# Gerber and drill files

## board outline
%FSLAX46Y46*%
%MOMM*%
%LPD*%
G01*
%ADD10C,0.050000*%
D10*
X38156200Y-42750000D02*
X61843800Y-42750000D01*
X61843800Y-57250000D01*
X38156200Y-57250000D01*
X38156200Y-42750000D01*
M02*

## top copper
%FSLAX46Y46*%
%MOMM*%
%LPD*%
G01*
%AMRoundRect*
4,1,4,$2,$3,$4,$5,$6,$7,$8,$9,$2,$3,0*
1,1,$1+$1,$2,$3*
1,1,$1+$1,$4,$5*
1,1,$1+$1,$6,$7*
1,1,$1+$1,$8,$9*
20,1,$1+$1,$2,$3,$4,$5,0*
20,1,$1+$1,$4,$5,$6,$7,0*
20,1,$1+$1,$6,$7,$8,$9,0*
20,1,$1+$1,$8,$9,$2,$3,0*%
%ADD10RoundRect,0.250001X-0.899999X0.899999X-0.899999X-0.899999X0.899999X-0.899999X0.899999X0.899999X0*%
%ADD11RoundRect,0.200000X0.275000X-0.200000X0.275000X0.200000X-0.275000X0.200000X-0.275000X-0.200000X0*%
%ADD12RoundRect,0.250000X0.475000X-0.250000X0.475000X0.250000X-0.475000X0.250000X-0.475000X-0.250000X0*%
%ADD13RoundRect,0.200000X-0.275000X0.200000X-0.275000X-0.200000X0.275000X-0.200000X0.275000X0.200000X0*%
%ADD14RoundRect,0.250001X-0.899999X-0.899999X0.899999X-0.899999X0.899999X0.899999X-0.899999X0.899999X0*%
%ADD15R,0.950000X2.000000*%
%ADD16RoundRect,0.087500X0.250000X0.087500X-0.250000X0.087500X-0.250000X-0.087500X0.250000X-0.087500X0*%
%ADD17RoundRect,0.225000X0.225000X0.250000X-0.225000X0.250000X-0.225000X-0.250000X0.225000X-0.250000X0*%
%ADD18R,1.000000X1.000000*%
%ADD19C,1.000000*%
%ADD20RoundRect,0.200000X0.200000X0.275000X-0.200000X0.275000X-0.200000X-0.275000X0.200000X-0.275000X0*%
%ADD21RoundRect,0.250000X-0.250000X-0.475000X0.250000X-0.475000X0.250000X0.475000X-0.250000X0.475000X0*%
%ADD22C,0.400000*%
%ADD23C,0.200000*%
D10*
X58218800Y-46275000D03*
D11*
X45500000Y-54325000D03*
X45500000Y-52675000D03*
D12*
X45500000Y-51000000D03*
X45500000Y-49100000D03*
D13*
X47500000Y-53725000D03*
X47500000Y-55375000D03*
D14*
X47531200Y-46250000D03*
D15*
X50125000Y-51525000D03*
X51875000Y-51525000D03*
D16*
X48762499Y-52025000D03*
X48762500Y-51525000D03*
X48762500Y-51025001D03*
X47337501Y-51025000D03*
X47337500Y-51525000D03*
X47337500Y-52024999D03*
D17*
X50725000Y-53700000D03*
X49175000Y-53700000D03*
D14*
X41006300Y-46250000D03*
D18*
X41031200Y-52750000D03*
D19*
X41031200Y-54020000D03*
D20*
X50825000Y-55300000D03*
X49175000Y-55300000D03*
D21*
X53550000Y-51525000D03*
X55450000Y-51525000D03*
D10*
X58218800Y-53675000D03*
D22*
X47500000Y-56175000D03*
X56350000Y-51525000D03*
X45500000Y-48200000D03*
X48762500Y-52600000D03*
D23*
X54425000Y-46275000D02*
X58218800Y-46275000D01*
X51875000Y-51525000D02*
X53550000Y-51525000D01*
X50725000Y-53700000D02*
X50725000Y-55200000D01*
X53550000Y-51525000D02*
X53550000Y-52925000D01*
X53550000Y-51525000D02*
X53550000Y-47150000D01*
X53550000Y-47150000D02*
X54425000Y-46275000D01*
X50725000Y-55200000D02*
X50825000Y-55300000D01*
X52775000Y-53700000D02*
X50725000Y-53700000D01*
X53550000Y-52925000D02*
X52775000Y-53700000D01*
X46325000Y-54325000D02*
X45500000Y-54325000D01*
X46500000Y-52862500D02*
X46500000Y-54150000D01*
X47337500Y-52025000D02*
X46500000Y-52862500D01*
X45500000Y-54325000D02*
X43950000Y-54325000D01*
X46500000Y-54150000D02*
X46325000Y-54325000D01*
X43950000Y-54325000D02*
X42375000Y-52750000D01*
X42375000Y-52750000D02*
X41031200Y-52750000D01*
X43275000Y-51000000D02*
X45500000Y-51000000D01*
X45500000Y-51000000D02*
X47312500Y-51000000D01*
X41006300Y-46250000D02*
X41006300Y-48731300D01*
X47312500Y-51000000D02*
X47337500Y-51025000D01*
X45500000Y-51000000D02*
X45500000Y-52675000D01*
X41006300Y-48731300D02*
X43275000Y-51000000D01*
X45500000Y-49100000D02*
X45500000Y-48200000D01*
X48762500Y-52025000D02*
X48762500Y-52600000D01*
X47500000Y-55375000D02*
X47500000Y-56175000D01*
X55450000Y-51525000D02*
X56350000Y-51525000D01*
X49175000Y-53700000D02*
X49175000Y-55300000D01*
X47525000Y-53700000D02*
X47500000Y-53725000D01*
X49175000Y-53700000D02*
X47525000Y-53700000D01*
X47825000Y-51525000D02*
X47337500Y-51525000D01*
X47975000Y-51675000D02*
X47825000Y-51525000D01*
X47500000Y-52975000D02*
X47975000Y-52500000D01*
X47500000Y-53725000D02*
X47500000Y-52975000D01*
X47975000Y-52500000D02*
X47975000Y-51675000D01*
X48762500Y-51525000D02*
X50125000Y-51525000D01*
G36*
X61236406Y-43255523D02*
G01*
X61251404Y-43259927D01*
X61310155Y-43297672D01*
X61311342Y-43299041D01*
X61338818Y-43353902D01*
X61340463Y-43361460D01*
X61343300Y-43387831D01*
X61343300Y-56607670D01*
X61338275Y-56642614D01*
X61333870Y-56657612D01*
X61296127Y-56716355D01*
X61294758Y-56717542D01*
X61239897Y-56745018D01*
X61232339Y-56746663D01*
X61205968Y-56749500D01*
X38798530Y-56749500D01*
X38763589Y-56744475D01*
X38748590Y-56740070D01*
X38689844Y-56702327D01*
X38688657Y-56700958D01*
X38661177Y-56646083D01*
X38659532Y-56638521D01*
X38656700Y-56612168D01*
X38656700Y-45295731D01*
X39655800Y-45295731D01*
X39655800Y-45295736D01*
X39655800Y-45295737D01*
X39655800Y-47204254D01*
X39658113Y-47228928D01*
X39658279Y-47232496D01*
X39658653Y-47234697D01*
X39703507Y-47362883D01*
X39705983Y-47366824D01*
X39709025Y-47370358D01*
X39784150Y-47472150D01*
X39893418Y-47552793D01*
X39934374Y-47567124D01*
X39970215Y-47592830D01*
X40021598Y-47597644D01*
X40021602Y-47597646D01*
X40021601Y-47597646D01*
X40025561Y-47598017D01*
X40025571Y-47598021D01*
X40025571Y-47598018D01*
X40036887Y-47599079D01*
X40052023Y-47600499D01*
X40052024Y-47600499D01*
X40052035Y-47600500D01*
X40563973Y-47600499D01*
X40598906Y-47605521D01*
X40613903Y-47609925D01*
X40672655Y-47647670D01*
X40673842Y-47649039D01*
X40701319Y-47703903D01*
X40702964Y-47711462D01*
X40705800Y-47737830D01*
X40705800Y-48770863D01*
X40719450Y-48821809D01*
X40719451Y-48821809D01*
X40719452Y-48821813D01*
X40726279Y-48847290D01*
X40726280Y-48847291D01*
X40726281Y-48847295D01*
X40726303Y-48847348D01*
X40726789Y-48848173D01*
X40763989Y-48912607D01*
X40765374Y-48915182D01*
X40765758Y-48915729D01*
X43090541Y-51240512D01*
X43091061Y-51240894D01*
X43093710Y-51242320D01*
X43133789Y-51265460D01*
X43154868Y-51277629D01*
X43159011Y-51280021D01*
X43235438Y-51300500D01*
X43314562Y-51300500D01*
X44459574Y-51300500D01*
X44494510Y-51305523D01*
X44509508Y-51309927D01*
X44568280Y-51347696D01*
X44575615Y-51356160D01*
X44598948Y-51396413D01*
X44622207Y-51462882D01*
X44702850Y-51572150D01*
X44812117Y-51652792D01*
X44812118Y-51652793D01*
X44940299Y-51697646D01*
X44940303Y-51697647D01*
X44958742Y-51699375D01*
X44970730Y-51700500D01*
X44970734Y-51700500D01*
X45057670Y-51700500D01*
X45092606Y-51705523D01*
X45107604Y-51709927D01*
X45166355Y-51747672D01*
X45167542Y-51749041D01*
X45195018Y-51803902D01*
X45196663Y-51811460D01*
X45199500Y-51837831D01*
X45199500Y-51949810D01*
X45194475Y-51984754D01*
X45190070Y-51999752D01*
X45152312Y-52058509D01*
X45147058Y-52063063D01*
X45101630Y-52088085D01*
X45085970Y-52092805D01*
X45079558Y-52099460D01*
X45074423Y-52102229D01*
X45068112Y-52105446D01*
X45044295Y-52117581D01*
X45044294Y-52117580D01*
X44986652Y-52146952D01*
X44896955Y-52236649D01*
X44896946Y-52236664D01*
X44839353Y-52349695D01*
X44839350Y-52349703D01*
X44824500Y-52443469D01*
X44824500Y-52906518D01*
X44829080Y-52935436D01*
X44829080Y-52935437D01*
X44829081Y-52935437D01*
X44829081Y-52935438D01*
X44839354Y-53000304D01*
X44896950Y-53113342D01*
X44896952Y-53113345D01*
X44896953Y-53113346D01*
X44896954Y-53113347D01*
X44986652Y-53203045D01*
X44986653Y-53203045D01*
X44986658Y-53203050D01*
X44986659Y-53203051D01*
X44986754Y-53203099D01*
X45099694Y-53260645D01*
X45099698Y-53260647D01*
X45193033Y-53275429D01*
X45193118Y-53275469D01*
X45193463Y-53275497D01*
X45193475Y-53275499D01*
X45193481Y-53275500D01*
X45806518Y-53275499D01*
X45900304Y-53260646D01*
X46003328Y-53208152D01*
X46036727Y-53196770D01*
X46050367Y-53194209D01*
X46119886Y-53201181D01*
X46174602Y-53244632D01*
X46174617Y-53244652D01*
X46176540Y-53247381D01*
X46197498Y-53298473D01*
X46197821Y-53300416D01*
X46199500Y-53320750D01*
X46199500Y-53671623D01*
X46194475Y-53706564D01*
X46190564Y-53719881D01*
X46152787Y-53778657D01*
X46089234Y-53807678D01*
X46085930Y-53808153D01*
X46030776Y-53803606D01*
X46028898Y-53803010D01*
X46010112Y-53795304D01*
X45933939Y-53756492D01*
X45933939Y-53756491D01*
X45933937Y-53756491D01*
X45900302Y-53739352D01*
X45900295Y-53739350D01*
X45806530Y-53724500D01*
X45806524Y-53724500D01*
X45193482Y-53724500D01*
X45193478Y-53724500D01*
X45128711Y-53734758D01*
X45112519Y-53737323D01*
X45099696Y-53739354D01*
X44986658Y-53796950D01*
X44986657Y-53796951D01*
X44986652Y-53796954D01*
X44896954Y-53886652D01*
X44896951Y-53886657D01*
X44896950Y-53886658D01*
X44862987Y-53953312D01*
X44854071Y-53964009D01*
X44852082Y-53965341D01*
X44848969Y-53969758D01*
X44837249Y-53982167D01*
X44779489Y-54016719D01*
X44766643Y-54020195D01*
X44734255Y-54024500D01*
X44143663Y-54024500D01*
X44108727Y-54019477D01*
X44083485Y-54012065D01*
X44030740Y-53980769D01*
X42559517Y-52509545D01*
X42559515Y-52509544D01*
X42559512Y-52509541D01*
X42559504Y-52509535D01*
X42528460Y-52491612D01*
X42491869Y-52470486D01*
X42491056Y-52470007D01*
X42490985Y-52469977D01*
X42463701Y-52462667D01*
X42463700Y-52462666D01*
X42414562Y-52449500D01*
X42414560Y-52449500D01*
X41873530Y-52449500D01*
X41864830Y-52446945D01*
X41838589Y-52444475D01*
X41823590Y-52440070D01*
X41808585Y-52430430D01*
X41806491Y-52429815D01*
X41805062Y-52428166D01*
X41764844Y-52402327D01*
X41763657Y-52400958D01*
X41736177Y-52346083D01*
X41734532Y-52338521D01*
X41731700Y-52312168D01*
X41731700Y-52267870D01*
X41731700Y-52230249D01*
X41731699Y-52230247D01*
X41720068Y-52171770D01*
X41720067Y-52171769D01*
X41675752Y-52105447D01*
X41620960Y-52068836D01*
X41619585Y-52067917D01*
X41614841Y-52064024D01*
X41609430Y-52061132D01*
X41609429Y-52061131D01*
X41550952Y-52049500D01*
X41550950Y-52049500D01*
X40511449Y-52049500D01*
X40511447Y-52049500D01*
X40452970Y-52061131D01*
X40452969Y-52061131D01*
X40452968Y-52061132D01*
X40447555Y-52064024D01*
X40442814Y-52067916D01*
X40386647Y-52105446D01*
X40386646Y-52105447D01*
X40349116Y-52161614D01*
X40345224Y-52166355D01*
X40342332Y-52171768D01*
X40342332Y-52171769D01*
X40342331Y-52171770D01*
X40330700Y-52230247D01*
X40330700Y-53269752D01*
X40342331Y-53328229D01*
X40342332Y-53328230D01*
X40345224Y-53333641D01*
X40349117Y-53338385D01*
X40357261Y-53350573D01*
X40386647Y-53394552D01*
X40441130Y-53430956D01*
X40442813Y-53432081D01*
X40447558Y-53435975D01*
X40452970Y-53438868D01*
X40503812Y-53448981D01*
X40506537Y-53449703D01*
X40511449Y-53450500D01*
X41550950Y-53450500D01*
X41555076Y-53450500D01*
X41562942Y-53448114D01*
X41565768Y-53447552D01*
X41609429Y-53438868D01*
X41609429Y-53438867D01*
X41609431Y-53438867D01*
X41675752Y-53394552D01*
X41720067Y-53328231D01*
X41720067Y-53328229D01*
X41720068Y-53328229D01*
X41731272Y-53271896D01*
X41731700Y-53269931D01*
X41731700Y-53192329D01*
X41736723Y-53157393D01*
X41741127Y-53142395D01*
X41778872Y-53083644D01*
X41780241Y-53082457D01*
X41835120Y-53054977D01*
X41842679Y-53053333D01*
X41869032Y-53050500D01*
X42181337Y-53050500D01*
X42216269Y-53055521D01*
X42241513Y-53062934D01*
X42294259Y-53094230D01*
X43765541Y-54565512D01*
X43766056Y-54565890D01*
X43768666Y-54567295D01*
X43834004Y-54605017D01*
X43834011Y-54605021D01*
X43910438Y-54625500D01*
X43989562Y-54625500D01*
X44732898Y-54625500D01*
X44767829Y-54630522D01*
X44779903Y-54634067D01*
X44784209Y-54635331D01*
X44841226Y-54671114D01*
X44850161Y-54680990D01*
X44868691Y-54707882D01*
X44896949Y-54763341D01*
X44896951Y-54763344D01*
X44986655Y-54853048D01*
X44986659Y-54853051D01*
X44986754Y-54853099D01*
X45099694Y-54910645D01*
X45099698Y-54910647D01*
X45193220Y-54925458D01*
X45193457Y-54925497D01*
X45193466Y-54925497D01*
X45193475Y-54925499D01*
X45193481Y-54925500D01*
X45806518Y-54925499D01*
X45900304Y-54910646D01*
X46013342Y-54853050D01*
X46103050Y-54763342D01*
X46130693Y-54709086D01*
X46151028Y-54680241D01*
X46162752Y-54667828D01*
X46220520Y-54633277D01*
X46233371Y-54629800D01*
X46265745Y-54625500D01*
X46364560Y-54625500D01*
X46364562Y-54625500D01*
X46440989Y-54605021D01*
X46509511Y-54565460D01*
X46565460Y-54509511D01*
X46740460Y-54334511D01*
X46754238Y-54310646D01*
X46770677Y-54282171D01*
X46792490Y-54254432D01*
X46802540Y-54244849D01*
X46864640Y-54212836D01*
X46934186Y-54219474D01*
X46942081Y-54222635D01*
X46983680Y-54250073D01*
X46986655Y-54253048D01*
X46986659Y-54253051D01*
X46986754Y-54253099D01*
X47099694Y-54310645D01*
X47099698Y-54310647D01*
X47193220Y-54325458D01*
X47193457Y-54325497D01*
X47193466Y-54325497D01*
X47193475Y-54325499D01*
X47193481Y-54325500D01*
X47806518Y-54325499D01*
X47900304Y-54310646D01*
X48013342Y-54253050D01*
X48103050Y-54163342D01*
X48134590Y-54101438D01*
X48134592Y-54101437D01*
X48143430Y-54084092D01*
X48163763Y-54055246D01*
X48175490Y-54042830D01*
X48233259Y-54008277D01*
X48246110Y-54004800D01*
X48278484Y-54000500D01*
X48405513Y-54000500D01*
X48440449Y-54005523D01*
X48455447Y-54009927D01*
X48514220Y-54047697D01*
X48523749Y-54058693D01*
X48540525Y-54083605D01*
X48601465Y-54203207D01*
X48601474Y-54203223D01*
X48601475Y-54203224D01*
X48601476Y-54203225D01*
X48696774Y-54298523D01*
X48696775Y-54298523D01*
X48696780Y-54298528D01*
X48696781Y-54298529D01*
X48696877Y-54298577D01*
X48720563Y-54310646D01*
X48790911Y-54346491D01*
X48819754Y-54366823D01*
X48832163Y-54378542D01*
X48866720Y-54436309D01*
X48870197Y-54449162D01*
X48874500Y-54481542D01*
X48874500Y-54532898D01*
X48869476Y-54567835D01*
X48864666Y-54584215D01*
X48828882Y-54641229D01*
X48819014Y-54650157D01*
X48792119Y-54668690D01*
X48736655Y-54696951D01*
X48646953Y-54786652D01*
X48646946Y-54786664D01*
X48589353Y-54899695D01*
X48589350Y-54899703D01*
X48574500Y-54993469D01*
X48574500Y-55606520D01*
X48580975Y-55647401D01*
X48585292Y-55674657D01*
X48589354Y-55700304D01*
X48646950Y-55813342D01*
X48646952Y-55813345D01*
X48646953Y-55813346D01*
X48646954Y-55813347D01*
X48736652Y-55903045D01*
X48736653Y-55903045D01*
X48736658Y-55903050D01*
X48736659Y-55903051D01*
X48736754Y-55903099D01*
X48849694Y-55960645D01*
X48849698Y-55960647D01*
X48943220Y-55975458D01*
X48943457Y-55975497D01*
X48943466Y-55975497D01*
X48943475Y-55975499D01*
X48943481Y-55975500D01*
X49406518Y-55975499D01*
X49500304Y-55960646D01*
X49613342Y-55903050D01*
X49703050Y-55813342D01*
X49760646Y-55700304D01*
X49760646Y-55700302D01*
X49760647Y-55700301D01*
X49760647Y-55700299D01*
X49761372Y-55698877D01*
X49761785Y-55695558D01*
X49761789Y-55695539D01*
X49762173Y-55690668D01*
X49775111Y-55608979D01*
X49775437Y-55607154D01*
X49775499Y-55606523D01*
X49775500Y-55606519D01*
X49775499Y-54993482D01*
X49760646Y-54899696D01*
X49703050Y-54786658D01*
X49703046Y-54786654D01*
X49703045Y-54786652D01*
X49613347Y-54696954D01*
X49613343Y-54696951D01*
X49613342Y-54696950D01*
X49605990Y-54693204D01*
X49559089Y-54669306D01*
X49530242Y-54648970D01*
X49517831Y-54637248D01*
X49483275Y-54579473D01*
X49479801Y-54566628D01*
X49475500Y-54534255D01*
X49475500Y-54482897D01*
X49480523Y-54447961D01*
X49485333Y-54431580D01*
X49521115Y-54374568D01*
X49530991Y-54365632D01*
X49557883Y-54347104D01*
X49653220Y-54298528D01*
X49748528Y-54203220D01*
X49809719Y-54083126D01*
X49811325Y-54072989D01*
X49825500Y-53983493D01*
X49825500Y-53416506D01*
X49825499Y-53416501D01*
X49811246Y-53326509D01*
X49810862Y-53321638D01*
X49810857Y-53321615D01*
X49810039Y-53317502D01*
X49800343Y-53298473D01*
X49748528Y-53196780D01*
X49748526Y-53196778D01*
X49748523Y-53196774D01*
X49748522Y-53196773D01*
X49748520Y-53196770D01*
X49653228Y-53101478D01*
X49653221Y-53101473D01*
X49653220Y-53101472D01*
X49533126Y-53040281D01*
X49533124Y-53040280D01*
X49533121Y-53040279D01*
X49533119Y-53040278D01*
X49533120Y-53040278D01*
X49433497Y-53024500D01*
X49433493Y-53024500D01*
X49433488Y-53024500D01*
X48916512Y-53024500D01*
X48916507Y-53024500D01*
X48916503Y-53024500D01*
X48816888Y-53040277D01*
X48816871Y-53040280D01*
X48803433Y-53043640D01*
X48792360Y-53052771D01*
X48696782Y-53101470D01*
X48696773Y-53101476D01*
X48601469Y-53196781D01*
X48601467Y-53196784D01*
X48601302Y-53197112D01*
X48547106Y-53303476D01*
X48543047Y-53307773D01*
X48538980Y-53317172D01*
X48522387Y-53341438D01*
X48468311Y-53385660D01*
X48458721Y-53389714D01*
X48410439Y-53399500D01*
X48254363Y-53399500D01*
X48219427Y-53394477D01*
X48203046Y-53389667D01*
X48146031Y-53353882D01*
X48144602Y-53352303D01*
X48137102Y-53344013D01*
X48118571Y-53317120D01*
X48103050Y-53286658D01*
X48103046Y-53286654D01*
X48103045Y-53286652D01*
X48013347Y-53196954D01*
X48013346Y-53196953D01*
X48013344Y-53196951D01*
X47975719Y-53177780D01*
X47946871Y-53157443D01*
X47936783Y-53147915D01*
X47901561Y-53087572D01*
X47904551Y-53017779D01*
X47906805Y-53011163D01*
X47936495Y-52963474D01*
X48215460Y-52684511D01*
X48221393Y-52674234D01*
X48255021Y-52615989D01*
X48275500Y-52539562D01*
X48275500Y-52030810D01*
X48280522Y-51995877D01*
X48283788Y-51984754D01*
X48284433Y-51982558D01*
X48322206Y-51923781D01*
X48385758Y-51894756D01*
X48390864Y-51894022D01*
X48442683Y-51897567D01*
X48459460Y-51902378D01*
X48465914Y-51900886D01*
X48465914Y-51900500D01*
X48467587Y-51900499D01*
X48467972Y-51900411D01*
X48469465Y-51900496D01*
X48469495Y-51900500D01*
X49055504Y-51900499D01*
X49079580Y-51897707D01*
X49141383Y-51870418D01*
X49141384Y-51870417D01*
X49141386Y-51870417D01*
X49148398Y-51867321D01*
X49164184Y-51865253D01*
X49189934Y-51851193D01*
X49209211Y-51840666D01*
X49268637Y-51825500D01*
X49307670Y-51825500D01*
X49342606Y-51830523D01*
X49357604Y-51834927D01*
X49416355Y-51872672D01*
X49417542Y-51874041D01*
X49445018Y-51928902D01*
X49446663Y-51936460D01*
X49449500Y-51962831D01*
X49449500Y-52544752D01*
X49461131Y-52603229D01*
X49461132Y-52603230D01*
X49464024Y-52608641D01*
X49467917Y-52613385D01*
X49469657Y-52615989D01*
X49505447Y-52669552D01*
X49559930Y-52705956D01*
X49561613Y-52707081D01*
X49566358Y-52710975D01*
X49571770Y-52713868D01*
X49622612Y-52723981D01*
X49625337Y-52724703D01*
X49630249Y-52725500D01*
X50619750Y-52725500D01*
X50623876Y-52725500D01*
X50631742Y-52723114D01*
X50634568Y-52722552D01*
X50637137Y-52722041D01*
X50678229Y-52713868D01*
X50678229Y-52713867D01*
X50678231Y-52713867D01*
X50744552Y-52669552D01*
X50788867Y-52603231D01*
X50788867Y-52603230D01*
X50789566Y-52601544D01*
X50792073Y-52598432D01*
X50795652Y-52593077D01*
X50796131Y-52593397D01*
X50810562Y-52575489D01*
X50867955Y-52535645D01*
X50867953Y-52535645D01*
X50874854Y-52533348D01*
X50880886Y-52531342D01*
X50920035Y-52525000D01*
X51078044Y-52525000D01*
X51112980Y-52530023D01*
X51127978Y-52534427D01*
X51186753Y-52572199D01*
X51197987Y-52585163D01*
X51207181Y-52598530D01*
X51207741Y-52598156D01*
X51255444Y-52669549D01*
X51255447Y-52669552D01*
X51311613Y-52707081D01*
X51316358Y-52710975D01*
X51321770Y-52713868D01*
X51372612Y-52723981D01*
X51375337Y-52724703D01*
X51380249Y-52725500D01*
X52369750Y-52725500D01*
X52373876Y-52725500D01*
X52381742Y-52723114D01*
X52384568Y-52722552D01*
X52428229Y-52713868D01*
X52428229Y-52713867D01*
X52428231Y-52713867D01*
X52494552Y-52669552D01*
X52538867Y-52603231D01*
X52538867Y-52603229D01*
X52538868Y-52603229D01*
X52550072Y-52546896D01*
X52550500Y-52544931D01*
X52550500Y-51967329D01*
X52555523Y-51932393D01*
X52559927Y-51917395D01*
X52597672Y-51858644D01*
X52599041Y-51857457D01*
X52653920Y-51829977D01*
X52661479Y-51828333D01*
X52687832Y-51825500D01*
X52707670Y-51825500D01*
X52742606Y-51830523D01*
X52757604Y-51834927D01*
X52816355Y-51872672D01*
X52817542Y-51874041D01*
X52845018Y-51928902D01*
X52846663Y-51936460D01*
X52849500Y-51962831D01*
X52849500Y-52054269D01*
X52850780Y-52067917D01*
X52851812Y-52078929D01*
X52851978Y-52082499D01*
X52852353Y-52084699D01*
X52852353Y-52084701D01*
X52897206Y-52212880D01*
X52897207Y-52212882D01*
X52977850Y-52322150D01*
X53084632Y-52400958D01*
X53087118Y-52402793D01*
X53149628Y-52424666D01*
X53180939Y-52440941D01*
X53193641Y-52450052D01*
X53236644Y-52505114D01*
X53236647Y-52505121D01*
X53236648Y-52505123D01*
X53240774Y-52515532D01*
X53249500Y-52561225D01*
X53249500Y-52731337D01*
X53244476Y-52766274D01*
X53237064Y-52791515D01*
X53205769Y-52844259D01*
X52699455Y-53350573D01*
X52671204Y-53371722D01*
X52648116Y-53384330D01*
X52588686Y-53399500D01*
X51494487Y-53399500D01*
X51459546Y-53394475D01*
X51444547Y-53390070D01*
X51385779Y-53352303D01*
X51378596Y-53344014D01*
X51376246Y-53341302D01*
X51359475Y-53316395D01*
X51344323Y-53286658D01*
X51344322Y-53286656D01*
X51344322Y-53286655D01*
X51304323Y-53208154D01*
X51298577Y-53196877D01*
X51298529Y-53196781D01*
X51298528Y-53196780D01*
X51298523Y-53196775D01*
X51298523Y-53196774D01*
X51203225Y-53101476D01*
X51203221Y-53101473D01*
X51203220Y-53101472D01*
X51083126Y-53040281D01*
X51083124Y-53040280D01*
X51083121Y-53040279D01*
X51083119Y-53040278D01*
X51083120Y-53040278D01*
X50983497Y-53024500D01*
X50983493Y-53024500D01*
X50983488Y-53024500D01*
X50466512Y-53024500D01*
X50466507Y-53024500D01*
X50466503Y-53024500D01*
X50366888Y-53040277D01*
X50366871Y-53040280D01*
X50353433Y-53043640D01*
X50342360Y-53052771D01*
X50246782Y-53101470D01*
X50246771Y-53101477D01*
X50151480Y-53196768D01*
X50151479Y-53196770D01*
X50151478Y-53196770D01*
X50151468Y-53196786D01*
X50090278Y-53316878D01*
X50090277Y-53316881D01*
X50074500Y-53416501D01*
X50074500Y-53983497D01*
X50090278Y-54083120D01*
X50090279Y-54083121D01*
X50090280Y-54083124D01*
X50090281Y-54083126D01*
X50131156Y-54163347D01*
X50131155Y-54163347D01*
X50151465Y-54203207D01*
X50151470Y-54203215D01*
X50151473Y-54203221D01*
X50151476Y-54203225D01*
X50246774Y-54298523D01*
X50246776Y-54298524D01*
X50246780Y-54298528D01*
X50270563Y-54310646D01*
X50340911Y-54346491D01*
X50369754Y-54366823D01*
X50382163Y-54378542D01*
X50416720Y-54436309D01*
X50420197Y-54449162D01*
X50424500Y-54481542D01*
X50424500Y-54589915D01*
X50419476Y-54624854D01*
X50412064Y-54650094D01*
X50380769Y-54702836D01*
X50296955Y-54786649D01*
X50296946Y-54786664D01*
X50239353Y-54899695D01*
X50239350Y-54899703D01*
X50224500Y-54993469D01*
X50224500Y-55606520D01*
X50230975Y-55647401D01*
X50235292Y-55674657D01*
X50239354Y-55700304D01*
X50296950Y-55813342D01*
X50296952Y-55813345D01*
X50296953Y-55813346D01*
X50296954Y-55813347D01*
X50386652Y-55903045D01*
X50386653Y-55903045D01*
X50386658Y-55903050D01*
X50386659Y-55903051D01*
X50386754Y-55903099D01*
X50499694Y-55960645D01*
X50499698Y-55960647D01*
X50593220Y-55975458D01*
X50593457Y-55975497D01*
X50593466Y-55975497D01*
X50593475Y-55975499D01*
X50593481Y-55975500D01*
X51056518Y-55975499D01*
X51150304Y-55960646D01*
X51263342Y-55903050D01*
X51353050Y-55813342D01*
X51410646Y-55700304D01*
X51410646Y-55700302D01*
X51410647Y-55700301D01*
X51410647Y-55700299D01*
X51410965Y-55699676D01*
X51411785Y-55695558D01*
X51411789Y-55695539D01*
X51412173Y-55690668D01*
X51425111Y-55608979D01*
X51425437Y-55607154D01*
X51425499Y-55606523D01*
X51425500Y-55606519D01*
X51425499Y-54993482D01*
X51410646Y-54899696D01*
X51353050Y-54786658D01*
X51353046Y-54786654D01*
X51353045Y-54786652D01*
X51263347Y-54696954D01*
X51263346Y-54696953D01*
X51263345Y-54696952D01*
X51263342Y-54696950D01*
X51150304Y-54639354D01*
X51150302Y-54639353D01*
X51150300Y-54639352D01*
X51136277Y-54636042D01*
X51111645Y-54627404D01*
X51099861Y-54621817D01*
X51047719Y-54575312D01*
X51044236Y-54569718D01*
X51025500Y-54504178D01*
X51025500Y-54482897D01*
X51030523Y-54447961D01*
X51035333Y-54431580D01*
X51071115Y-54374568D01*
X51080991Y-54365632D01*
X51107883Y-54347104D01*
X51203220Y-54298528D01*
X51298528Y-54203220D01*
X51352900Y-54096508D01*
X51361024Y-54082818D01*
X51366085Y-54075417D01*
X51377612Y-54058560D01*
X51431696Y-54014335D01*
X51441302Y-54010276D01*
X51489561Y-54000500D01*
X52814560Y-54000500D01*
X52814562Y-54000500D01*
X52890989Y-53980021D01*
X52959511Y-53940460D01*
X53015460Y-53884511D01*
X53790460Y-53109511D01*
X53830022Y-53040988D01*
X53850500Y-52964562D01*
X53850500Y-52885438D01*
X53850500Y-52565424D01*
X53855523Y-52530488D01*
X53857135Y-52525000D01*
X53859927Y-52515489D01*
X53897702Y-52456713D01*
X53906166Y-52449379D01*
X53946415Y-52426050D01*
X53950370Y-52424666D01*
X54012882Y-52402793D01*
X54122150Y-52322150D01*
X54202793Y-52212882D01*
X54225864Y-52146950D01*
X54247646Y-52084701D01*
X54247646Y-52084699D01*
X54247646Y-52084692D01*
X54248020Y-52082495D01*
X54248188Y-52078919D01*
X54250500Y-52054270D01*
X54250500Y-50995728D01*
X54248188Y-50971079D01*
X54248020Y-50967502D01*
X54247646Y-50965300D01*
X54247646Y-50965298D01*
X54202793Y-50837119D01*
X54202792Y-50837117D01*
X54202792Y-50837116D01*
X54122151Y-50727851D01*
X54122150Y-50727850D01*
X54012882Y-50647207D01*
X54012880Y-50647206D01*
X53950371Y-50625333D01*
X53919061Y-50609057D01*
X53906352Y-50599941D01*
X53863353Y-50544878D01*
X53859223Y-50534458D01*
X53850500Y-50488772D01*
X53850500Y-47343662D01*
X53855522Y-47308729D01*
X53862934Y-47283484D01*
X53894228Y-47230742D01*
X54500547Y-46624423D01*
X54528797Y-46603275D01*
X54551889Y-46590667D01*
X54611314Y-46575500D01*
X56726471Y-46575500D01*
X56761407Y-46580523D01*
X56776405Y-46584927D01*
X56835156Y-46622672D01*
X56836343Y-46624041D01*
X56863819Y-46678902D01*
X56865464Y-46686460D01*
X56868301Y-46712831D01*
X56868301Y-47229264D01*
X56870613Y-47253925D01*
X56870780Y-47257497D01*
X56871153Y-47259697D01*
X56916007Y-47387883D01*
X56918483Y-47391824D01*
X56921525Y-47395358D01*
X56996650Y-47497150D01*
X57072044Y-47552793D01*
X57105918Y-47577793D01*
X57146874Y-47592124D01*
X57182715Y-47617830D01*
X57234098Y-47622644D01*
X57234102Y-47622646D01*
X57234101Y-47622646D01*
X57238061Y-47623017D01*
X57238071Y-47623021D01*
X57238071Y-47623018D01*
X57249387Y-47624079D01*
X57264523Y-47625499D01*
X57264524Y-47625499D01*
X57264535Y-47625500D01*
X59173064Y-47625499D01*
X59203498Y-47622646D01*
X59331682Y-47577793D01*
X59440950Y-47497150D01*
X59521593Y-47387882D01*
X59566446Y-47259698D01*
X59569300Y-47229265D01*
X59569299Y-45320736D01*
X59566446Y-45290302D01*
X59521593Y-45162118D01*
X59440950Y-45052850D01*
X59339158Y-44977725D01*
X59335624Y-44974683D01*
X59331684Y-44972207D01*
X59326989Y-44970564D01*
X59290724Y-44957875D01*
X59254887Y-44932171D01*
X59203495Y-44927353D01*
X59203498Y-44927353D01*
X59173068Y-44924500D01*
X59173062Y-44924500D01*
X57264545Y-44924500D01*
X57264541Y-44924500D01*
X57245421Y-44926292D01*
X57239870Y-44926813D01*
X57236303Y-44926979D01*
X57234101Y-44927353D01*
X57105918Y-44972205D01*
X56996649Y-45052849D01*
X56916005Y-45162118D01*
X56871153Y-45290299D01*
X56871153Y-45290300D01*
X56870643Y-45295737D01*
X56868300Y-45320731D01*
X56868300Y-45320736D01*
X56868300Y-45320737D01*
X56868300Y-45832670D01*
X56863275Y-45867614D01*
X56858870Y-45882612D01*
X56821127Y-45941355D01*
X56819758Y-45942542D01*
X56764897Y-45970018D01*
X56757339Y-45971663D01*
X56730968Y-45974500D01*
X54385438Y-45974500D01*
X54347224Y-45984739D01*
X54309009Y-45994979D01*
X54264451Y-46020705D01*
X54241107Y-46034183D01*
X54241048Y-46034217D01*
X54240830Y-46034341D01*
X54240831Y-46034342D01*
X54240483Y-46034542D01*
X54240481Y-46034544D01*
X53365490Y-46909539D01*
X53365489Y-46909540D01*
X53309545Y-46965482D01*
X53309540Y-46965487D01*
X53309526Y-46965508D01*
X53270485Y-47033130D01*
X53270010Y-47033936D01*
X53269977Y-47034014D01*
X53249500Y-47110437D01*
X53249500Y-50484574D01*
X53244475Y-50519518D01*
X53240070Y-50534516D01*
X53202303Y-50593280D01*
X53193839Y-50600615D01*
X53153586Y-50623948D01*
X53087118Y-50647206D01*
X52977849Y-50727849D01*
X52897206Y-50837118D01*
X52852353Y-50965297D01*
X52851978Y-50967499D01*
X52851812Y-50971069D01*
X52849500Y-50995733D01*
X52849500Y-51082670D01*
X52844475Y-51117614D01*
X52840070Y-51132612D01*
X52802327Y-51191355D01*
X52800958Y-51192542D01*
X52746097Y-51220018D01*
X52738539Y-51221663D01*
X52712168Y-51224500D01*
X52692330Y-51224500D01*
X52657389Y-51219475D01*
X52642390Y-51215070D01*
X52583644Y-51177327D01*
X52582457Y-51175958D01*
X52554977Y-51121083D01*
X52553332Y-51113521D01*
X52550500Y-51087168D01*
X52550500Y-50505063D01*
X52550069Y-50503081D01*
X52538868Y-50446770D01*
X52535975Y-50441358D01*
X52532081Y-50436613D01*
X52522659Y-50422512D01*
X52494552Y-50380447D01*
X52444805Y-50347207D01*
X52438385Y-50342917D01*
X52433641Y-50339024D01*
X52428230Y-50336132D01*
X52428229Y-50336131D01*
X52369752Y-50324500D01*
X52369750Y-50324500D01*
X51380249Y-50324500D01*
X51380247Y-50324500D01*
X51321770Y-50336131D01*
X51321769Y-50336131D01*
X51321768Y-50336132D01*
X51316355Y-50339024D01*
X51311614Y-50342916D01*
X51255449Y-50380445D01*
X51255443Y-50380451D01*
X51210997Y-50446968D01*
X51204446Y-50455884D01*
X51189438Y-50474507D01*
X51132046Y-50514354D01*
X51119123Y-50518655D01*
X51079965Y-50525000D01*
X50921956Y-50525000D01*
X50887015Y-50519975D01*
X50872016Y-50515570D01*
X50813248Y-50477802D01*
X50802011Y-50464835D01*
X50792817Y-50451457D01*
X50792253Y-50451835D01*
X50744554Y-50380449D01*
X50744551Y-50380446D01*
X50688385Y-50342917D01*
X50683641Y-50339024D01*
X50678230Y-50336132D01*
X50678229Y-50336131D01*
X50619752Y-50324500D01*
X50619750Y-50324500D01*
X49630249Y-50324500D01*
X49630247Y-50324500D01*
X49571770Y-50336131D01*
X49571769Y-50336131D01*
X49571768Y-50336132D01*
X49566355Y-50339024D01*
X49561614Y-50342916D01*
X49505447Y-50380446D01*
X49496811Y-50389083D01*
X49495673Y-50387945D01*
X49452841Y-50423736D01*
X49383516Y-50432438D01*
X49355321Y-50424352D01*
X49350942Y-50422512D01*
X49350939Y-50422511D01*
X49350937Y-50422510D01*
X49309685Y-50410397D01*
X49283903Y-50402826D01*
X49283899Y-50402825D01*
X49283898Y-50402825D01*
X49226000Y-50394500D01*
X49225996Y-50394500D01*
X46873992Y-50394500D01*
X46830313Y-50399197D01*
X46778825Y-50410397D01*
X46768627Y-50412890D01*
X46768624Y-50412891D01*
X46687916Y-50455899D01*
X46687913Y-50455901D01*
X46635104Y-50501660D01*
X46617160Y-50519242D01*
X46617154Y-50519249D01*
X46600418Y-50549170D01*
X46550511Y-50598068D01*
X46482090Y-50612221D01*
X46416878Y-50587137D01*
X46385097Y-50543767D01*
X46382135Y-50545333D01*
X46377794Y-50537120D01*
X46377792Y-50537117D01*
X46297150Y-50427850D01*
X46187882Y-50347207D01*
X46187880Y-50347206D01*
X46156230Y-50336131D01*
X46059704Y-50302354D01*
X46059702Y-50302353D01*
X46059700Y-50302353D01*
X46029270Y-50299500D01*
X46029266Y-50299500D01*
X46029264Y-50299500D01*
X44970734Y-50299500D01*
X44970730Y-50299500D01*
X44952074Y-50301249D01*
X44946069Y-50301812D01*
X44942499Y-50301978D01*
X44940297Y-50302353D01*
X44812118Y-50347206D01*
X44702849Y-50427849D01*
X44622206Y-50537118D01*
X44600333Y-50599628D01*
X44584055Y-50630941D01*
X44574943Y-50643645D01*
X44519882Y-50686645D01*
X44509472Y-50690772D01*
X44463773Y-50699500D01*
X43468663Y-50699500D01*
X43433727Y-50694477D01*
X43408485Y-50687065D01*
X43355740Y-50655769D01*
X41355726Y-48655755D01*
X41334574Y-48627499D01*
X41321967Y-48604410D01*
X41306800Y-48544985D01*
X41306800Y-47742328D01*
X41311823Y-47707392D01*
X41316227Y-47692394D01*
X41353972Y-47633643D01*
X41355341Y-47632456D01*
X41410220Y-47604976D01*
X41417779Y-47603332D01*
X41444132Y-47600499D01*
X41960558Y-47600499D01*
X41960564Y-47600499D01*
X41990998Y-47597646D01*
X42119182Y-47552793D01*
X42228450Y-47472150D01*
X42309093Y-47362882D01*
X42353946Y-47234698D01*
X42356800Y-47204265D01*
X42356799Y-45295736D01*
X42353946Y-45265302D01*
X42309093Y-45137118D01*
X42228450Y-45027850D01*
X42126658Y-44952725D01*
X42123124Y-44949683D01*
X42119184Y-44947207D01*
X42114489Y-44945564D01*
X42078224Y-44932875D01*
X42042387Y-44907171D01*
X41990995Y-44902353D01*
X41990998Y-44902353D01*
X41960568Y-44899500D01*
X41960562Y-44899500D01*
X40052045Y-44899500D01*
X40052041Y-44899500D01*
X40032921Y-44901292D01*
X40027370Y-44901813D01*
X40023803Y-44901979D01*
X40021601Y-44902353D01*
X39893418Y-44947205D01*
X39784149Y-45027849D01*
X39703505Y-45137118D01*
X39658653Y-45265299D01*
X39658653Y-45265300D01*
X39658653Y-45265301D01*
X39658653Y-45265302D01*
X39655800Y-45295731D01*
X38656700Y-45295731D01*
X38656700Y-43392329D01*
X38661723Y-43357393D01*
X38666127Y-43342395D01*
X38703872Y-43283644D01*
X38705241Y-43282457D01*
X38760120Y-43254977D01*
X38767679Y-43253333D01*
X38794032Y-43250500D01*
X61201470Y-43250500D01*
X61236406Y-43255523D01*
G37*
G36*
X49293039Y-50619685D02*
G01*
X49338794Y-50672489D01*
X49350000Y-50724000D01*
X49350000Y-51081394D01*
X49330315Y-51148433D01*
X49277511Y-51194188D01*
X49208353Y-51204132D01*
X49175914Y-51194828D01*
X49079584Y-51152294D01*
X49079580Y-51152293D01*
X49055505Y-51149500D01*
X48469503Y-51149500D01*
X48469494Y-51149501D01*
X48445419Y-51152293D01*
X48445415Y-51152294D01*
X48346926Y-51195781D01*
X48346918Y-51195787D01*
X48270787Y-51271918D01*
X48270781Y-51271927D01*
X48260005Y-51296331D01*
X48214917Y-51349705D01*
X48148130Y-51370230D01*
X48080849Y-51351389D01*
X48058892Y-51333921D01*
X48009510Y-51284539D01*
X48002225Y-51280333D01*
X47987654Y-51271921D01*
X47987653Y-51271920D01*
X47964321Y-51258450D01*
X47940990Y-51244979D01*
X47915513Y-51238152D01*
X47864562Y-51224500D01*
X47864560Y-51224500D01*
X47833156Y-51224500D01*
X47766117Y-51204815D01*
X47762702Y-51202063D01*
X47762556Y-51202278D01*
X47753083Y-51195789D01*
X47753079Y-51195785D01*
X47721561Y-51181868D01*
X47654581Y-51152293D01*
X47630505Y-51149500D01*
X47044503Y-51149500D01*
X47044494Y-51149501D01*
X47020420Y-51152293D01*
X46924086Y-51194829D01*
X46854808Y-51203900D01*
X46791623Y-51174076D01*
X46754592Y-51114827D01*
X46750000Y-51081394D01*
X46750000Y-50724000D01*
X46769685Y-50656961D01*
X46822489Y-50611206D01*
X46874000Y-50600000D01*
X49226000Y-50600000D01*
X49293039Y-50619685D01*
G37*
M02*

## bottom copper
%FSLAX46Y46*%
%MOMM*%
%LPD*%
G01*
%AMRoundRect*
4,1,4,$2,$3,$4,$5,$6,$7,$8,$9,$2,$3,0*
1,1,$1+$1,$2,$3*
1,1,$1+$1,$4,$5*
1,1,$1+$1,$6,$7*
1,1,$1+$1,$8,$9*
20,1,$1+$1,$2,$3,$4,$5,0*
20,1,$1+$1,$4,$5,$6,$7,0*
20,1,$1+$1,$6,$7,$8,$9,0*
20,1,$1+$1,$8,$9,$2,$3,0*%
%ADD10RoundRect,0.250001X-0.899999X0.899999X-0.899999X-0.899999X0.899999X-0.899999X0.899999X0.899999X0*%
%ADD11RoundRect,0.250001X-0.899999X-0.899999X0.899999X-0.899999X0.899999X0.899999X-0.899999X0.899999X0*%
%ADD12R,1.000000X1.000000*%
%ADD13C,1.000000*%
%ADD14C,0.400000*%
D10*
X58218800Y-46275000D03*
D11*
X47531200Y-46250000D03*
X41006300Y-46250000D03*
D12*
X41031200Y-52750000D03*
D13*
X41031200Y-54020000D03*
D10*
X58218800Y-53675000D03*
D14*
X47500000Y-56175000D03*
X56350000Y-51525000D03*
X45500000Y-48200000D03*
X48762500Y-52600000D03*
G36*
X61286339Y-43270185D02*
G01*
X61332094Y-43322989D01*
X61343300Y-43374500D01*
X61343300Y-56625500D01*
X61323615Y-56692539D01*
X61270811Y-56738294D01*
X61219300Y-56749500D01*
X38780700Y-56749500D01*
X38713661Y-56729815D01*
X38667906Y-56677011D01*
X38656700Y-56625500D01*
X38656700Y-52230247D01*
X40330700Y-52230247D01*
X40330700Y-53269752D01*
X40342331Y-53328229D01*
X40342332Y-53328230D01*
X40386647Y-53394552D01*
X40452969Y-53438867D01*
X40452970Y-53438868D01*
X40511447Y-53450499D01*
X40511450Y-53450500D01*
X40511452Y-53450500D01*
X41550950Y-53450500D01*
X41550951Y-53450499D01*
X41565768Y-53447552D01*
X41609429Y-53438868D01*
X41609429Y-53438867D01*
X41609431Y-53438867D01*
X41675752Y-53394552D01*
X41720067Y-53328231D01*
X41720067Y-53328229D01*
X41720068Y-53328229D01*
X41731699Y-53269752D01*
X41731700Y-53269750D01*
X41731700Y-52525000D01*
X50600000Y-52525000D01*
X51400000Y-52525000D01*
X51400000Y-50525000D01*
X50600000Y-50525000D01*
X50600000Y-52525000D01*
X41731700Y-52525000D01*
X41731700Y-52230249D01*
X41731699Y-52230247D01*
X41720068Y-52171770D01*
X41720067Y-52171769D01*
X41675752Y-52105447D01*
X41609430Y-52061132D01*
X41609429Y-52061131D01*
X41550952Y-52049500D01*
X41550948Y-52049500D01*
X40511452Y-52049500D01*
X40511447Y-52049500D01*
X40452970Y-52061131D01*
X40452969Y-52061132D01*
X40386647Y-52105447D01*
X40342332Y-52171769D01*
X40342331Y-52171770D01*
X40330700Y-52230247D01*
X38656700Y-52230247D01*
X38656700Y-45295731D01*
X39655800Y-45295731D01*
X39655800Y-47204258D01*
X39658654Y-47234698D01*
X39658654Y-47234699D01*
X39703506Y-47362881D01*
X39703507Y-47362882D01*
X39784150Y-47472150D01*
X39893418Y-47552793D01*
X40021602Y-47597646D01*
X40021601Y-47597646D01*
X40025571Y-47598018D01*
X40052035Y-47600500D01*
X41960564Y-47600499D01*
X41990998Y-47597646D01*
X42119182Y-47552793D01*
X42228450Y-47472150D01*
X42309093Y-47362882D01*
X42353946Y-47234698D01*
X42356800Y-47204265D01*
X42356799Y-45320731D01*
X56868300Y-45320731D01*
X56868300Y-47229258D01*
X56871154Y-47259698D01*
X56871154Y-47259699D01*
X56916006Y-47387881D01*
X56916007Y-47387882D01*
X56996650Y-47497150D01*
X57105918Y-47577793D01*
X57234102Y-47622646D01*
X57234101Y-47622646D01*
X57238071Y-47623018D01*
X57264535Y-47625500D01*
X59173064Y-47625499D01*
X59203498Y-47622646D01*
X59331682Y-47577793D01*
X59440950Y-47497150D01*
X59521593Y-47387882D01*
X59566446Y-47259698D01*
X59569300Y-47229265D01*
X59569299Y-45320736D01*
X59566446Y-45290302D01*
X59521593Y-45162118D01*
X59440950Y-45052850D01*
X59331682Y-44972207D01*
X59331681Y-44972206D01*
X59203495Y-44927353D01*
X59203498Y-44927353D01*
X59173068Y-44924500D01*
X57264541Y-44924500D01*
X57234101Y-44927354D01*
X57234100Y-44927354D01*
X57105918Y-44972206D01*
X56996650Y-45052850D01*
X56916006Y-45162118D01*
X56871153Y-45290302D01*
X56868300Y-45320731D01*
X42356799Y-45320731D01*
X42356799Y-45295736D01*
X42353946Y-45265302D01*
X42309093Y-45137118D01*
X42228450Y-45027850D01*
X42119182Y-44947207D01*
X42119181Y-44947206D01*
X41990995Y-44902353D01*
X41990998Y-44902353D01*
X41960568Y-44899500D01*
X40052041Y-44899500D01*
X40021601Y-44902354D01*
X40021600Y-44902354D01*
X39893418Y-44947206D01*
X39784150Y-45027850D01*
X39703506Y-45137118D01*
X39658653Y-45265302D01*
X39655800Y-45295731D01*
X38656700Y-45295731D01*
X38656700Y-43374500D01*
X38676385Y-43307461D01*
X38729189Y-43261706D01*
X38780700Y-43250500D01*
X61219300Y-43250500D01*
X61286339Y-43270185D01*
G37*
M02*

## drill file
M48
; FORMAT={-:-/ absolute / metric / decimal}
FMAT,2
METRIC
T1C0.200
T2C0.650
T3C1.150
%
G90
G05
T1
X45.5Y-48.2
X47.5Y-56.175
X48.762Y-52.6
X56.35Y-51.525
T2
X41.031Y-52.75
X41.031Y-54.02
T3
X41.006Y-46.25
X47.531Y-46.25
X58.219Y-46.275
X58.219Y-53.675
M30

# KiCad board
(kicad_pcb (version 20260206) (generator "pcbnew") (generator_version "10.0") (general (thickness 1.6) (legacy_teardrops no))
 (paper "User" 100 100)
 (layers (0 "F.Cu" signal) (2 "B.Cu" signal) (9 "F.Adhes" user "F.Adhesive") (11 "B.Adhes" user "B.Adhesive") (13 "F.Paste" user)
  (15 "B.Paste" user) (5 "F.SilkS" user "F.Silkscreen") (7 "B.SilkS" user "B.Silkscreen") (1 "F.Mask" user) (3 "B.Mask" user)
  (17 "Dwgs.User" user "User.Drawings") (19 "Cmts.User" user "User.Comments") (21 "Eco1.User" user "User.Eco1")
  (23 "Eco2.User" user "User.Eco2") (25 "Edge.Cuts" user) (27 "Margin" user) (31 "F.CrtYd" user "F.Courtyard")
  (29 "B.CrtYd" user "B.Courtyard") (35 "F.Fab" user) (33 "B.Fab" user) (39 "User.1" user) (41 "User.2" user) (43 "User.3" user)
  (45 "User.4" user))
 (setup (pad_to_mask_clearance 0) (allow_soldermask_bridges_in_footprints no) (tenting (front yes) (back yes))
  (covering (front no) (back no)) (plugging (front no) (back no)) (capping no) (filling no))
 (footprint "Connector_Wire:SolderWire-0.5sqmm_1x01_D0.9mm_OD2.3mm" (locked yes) (layer "F.Cu") (at 58.2188 46.275 -90)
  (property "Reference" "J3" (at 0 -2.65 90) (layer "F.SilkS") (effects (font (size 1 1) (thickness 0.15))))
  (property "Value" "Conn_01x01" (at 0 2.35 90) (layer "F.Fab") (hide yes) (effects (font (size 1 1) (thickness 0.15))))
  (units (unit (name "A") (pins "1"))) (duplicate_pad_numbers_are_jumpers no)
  (pad "1" thru_hole roundrect (at 0 0 270) (size 2.3 2.3) (drill 1.15) (layers "*.Cu" "*.Mask") (remove_unused_layers no)
   (roundrect_rratio 0.108696) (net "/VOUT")))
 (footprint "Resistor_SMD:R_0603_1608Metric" (layer "F.Cu") (at 45.5 53.5 90)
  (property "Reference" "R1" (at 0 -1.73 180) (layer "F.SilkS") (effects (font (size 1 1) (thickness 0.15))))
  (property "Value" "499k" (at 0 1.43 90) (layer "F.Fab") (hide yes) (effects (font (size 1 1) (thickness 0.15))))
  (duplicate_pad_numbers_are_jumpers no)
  (pad "1" smd roundrect (at -0.825 0 90) (size 0.8 0.95) (layers "F.Cu" "F.Mask" "F.Paste") (roundrect_rratio 0.25) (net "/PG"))
  (pad "2" smd roundrect (at 0.825 0 90) (size 0.8 0.95) (layers "F.Cu" "F.Mask" "F.Paste") (roundrect_rratio 0.25) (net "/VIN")))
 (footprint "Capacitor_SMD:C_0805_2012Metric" (layer "F.Cu") (at 45.5 50.05 90)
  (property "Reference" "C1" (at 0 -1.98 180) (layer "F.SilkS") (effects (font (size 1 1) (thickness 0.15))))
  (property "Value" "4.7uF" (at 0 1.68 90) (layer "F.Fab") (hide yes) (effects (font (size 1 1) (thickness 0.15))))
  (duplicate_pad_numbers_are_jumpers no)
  (pad "1" smd roundrect (at -0.95 0 90) (size 1 1.45) (layers "F.Cu" "F.Mask" "F.Paste") (roundrect_rratio 0.25) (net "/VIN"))
  (pad "2" smd roundrect (at 0.95 0 90) (size 1 1.45) (layers "F.Cu" "F.Mask" "F.Paste") (roundrect_rratio 0.25) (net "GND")))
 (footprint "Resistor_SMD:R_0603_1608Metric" (layer "F.Cu") (at 47.5 54.55 -90)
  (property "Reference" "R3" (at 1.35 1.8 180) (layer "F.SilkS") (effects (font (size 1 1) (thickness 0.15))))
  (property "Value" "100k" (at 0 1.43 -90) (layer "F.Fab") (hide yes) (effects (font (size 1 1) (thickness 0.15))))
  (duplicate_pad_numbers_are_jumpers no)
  (pad "1" smd roundrect (at -0.825 0 -90) (size 0.8 0.95) (layers "F.Cu" "F.Mask" "F.Paste") (roundrect_rratio 0.25) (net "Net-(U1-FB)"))
  (pad "2" smd roundrect (at 0.825 0 -90) (size 0.8 0.95) (layers "F.Cu" "F.Mask" "F.Paste") (roundrect_rratio 0.25) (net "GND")))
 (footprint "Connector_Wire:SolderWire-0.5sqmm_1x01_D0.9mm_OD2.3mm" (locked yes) (layer "F.Cu") (at 47.5312 46.25)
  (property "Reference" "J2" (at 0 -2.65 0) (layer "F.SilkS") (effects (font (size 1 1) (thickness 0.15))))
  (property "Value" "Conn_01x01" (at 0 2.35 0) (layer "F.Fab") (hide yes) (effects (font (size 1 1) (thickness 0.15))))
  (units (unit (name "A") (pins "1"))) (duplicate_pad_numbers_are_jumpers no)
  (pad "1" thru_hole roundrect (at 0 0) (size 2.3 2.3) (drill 1.15) (layers "*.Cu" "*.Mask") (remove_unused_layers no)
   (roundrect_rratio 0.108696) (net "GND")))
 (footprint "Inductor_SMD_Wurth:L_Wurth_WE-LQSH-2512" (layer "F.Cu") (at 51 51.525)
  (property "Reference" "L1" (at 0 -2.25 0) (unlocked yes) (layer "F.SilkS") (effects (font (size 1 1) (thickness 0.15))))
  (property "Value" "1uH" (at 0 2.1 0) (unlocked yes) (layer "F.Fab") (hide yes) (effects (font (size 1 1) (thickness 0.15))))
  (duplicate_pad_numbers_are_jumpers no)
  (pad "1" smd rect (at -0.875 0) (size 0.95 2) (layers "F.Cu" "F.Mask" "F.Paste") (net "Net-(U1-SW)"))
  (pad "2" smd rect (at 0.875 0) (size 0.95 2) (layers "F.Cu" "F.Mask" "F.Paste") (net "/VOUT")))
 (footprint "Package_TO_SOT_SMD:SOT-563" (layer "F.Cu") (at 48.05 51.525 180)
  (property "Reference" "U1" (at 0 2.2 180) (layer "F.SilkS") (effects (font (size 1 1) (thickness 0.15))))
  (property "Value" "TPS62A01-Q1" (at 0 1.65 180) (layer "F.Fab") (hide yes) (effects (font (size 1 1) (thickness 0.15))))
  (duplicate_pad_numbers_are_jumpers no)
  (pad "1" smd roundrect (at -0.712499 -0.5 180) (size 0.675 0.35) (layers "F.Cu" "F.Mask" "F.Paste") (roundrect_rratio 0.25) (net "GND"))
  (pad "2" smd roundrect (at -0.7125 0 180) (size 0.675 0.35) (layers "F.Cu" "F.Mask" "F.Paste") (roundrect_rratio 0.25) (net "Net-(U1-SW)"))
  (pad "3" smd roundrect (at -0.7125 0.499999 180) (size 0.675 0.35) (layers "F.Cu" "F.Mask" "F.Paste") (roundrect_rratio 0.25) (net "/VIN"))
  (pad "4" smd roundrect (at 0.712499 0.5 180) (size 0.675 0.35) (layers "F.Cu" "F.Mask" "F.Paste") (roundrect_rratio 0.25) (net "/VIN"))
  (pad "5" smd roundrect (at 0.7125 0 180) (size 0.675 0.35) (layers "F.Cu" "F.Mask" "F.Paste") (roundrect_rratio 0.25) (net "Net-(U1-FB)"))
  (pad "6" smd roundrect (at 0.7125 -0.499999 180) (size 0.675 0.35) (layers "F.Cu" "F.Mask" "F.Paste") (roundrect_rratio 0.25) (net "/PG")))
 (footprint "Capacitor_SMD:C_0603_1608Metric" (layer "F.Cu") (at 49.95 53.7 180)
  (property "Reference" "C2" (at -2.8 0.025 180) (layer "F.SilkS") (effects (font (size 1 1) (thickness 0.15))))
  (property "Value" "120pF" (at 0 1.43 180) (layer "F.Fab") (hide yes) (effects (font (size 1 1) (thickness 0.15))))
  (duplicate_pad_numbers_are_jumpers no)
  (pad "1" smd roundrect (at -0.775 0 180) (size 0.9 0.95) (layers "F.Cu" "F.Mask" "F.Paste") (roundrect_rratio 0.25) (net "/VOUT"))
  (pad "2" smd roundrect (at 0.775 0 180) (size 0.9 0.95) (layers "F.Cu" "F.Mask" "F.Paste") (roundrect_rratio 0.25) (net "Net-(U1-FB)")))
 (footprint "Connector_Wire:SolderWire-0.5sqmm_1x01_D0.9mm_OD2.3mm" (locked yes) (layer "F.Cu") (at 41.0063 46.25)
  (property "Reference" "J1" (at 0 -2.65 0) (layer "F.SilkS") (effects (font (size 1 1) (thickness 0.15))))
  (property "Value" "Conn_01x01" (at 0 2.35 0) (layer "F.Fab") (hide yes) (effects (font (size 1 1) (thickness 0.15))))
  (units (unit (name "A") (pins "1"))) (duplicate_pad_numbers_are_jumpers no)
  (pad "1" thru_hole roundrect (at 0 0) (size 2.3 2.3) (drill 1.15) (layers "*.Cu" "*.Mask") (remove_unused_layers no)
   (roundrect_rratio 0.108696) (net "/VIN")))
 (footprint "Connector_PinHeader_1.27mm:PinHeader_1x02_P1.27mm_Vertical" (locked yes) (layer "F.Cu") (at 41.0312 53.385)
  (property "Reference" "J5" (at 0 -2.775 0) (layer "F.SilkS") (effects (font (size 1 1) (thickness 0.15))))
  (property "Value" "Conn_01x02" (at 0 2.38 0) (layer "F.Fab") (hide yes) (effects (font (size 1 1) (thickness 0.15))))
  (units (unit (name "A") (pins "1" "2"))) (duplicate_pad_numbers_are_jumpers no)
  (pad "1" thru_hole rect (at 0 -0.635) (size 1 1) (drill 0.65) (layers "*.Cu" "*.Mask") (remove_unused_layers no) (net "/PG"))
  (pad "2" thru_hole circle (at 0 0.635) (size 1 1) (drill 0.65) (layers "*.Cu" "*.Mask") (remove_unused_layers no) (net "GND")))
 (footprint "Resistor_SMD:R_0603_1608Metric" (layer "F.Cu") (at 50 55.3 180)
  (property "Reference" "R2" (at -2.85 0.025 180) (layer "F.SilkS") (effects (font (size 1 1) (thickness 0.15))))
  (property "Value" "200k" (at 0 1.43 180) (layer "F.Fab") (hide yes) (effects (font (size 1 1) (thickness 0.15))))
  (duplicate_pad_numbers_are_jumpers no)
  (pad "1" smd roundrect (at -0.825 0 180) (size 0.8 0.95) (layers "F.Cu" "F.Mask" "F.Paste") (roundrect_rratio 0.25) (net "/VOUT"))
  (pad "2" smd roundrect (at 0.825 0 180) (size 0.8 0.95) (layers "F.Cu" "F.Mask" "F.Paste") (roundrect_rratio 0.25) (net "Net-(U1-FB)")))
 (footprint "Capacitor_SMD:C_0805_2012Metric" (layer "F.Cu") (at 54.5 51.525)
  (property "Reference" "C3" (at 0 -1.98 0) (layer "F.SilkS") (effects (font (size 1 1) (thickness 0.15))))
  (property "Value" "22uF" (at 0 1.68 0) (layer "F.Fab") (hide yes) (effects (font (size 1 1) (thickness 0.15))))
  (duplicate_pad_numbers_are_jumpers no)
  (pad "1" smd roundrect (at -0.95 0) (size 1 1.45) (layers "F.Cu" "F.Mask" "F.Paste") (roundrect_rratio 0.25) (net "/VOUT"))
  (pad "2" smd roundrect (at 0.95 0) (size 1 1.45) (layers "F.Cu" "F.Mask" "F.Paste") (roundrect_rratio 0.25) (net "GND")))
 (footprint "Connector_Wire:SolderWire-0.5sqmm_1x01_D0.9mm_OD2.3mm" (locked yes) (layer "F.Cu") (at 58.2188 53.675 -90)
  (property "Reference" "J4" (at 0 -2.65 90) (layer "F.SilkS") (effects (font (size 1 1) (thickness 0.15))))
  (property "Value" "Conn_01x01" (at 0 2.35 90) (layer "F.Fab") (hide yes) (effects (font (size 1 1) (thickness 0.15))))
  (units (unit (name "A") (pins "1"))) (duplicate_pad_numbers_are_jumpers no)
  (pad "1" thru_hole roundrect (at 0 0 270) (size 2.3 2.3) (drill 1.15) (layers "*.Cu" "*.Mask") (remove_unused_layers no)
   (roundrect_rratio 0.108696) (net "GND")))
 (gr_rect (start 38.1562 42.75) (end 61.8438 57.25) (stroke (width 0.05) (type solid)) (fill no) (locked yes) (layer "Edge.Cuts"))
 (segment (start 54.425 46.275) (end 58.2188 46.275) (width 0.2) (layer "F.Cu") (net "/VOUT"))
 (segment (start 51.875 51.525) (end 53.55 51.525) (width 0.2) (layer "F.Cu") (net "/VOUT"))
 (segment (start 50.725 53.7) (end 50.725 55.2) (width 0.2) (layer "F.Cu") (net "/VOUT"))
 (segment (start 53.55 51.525) (end 53.55 52.925) (width 0.2) (layer "F.Cu") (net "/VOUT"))
 (segment (start 53.55 51.525) (end 53.55 47.15) (width 0.2) (layer "F.Cu") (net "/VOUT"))
 (segment (start 53.55 47.15) (end 54.425 46.275) (width 0.2) (layer "F.Cu") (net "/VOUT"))
 (segment (start 50.725 55.2) (end 50.825 55.3) (width 0.2) (layer "F.Cu") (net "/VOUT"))
 (segment (start 52.775 53.7) (end 50.725 53.7) (width 0.2) (layer "F.Cu") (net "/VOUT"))
 (segment (start 53.55 52.925) (end 52.775 53.7) (width 0.2) (layer "F.Cu") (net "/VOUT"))
 (segment (start 46.325 54.325) (end 45.5 54.325) (width 0.2) (layer "F.Cu") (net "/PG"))
 (segment (start 46.5 52.8625) (end 46.5 54.15) (width 0.2) (layer "F.Cu") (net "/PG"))
 (segment (start 47.3375 52.025) (end 46.5 52.8625) (width 0.2) (layer "F.Cu") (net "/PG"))
 (segment (start 45.5 54.325) (end 43.95 54.325) (width 0.2) (layer "F.Cu") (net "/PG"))
 (segment (start 46.5 54.15) (end 46.325 54.325) (width 0.2) (layer "F.Cu") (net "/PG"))
 (segment (start 43.95 54.325) (end 42.375 52.75) (width 0.2) (layer "F.Cu") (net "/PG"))
 (segment (start 42.375 52.75) (end 41.0312 52.75) (width 0.2) (layer "F.Cu") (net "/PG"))
 (segment (start 43.275 51) (end 45.5 51) (width 0.2) (layer "F.Cu") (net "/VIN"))
 (segment (start 45.5 51) (end 47.3125 51) (width 0.2) (layer "F.Cu") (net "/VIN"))
 (segment (start 41.0063 46.25) (end 41.0063 48.7313) (width 0.2) (layer "F.Cu") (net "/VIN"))
 (segment (start 47.3125 51) (end 47.3375 51.025) (width 0.2) (layer "F.Cu") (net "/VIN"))
 (segment (start 45.5 51) (end 45.5 52.675) (width 0.2) (layer "F.Cu") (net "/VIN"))
 (segment (start 41.0063 48.7313) (end 43.275 51) (width 0.2) (layer "F.Cu") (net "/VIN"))
 (segment (start 45.5 49.1) (end 45.5 48.2) (width 0.2) (layer "F.Cu") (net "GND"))
 (segment (start 48.7625 52.025) (end 48.7625 52.6) (width 0.2) (layer "F.Cu") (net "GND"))
 (segment (start 47.5 55.375) (end 47.5 56.175) (width 0.2) (layer "F.Cu") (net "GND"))
 (segment (start 55.45 51.525) (end 56.35 51.525) (width 0.2) (layer "F.Cu") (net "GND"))
 (via (at 47.5 56.175) (size 0.4) (drill 0.2) (layers "F.Cu" "B.Cu") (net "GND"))
 (via (at 56.35 51.525) (size 0.4) (drill 0.2) (layers "F.Cu" "B.Cu") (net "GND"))
 (via (at 45.5 48.2) (size 0.4) (drill 0.2) (layers "F.Cu" "B.Cu") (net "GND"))
 (via (at 48.7625 52.6) (size 0.4) (drill 0.2) (layers "F.Cu" "B.Cu") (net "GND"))
 (segment (start 49.175 53.7) (end 49.175 55.3) (width 0.2) (layer "F.Cu") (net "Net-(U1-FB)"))
 (segment (start 47.525 53.7) (end 47.5 53.725) (width 0.2) (layer "F.Cu") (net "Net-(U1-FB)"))
 (segment (start 49.175 53.7) (end 47.525 53.7) (width 0.2) (layer "F.Cu") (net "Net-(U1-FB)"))
 (segment (start 47.825 51.525) (end 47.3375 51.525) (width 0.2) (layer "F.Cu") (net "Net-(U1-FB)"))
 (segment (start 47.975 51.675) (end 47.825 51.525) (width 0.2) (layer "F.Cu") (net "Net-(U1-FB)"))
 (segment (start 47.5 52.975) (end 47.975 52.5) (width 0.2) (layer "F.Cu") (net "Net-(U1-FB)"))
 (segment (start 47.5 53.725) (end 47.5 52.975) (width 0.2) (layer "F.Cu") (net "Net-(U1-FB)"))
 (segment (start 47.975 52.5) (end 47.975 51.675) (width 0.2) (layer "F.Cu") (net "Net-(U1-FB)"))
 (segment (start 48.7625 51.525) (end 50.125 51.525) (width 0.2) (layer "F.Cu") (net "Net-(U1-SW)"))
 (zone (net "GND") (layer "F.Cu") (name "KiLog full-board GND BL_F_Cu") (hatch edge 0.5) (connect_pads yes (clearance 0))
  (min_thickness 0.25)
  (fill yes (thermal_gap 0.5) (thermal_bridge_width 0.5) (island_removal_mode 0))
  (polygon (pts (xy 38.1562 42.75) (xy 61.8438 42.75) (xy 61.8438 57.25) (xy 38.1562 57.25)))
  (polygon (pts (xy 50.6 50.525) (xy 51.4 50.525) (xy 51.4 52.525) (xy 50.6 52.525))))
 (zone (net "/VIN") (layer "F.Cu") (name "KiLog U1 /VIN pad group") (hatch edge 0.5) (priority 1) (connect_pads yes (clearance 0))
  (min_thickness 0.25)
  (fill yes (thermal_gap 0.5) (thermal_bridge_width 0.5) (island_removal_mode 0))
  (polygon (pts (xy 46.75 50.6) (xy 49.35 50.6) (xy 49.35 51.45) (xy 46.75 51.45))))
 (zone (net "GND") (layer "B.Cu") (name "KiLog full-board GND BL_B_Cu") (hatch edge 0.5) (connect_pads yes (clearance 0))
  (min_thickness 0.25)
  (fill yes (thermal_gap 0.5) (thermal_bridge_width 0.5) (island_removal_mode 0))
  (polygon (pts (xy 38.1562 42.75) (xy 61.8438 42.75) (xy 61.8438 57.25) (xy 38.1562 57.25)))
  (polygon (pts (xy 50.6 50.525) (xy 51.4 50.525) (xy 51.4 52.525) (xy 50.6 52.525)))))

